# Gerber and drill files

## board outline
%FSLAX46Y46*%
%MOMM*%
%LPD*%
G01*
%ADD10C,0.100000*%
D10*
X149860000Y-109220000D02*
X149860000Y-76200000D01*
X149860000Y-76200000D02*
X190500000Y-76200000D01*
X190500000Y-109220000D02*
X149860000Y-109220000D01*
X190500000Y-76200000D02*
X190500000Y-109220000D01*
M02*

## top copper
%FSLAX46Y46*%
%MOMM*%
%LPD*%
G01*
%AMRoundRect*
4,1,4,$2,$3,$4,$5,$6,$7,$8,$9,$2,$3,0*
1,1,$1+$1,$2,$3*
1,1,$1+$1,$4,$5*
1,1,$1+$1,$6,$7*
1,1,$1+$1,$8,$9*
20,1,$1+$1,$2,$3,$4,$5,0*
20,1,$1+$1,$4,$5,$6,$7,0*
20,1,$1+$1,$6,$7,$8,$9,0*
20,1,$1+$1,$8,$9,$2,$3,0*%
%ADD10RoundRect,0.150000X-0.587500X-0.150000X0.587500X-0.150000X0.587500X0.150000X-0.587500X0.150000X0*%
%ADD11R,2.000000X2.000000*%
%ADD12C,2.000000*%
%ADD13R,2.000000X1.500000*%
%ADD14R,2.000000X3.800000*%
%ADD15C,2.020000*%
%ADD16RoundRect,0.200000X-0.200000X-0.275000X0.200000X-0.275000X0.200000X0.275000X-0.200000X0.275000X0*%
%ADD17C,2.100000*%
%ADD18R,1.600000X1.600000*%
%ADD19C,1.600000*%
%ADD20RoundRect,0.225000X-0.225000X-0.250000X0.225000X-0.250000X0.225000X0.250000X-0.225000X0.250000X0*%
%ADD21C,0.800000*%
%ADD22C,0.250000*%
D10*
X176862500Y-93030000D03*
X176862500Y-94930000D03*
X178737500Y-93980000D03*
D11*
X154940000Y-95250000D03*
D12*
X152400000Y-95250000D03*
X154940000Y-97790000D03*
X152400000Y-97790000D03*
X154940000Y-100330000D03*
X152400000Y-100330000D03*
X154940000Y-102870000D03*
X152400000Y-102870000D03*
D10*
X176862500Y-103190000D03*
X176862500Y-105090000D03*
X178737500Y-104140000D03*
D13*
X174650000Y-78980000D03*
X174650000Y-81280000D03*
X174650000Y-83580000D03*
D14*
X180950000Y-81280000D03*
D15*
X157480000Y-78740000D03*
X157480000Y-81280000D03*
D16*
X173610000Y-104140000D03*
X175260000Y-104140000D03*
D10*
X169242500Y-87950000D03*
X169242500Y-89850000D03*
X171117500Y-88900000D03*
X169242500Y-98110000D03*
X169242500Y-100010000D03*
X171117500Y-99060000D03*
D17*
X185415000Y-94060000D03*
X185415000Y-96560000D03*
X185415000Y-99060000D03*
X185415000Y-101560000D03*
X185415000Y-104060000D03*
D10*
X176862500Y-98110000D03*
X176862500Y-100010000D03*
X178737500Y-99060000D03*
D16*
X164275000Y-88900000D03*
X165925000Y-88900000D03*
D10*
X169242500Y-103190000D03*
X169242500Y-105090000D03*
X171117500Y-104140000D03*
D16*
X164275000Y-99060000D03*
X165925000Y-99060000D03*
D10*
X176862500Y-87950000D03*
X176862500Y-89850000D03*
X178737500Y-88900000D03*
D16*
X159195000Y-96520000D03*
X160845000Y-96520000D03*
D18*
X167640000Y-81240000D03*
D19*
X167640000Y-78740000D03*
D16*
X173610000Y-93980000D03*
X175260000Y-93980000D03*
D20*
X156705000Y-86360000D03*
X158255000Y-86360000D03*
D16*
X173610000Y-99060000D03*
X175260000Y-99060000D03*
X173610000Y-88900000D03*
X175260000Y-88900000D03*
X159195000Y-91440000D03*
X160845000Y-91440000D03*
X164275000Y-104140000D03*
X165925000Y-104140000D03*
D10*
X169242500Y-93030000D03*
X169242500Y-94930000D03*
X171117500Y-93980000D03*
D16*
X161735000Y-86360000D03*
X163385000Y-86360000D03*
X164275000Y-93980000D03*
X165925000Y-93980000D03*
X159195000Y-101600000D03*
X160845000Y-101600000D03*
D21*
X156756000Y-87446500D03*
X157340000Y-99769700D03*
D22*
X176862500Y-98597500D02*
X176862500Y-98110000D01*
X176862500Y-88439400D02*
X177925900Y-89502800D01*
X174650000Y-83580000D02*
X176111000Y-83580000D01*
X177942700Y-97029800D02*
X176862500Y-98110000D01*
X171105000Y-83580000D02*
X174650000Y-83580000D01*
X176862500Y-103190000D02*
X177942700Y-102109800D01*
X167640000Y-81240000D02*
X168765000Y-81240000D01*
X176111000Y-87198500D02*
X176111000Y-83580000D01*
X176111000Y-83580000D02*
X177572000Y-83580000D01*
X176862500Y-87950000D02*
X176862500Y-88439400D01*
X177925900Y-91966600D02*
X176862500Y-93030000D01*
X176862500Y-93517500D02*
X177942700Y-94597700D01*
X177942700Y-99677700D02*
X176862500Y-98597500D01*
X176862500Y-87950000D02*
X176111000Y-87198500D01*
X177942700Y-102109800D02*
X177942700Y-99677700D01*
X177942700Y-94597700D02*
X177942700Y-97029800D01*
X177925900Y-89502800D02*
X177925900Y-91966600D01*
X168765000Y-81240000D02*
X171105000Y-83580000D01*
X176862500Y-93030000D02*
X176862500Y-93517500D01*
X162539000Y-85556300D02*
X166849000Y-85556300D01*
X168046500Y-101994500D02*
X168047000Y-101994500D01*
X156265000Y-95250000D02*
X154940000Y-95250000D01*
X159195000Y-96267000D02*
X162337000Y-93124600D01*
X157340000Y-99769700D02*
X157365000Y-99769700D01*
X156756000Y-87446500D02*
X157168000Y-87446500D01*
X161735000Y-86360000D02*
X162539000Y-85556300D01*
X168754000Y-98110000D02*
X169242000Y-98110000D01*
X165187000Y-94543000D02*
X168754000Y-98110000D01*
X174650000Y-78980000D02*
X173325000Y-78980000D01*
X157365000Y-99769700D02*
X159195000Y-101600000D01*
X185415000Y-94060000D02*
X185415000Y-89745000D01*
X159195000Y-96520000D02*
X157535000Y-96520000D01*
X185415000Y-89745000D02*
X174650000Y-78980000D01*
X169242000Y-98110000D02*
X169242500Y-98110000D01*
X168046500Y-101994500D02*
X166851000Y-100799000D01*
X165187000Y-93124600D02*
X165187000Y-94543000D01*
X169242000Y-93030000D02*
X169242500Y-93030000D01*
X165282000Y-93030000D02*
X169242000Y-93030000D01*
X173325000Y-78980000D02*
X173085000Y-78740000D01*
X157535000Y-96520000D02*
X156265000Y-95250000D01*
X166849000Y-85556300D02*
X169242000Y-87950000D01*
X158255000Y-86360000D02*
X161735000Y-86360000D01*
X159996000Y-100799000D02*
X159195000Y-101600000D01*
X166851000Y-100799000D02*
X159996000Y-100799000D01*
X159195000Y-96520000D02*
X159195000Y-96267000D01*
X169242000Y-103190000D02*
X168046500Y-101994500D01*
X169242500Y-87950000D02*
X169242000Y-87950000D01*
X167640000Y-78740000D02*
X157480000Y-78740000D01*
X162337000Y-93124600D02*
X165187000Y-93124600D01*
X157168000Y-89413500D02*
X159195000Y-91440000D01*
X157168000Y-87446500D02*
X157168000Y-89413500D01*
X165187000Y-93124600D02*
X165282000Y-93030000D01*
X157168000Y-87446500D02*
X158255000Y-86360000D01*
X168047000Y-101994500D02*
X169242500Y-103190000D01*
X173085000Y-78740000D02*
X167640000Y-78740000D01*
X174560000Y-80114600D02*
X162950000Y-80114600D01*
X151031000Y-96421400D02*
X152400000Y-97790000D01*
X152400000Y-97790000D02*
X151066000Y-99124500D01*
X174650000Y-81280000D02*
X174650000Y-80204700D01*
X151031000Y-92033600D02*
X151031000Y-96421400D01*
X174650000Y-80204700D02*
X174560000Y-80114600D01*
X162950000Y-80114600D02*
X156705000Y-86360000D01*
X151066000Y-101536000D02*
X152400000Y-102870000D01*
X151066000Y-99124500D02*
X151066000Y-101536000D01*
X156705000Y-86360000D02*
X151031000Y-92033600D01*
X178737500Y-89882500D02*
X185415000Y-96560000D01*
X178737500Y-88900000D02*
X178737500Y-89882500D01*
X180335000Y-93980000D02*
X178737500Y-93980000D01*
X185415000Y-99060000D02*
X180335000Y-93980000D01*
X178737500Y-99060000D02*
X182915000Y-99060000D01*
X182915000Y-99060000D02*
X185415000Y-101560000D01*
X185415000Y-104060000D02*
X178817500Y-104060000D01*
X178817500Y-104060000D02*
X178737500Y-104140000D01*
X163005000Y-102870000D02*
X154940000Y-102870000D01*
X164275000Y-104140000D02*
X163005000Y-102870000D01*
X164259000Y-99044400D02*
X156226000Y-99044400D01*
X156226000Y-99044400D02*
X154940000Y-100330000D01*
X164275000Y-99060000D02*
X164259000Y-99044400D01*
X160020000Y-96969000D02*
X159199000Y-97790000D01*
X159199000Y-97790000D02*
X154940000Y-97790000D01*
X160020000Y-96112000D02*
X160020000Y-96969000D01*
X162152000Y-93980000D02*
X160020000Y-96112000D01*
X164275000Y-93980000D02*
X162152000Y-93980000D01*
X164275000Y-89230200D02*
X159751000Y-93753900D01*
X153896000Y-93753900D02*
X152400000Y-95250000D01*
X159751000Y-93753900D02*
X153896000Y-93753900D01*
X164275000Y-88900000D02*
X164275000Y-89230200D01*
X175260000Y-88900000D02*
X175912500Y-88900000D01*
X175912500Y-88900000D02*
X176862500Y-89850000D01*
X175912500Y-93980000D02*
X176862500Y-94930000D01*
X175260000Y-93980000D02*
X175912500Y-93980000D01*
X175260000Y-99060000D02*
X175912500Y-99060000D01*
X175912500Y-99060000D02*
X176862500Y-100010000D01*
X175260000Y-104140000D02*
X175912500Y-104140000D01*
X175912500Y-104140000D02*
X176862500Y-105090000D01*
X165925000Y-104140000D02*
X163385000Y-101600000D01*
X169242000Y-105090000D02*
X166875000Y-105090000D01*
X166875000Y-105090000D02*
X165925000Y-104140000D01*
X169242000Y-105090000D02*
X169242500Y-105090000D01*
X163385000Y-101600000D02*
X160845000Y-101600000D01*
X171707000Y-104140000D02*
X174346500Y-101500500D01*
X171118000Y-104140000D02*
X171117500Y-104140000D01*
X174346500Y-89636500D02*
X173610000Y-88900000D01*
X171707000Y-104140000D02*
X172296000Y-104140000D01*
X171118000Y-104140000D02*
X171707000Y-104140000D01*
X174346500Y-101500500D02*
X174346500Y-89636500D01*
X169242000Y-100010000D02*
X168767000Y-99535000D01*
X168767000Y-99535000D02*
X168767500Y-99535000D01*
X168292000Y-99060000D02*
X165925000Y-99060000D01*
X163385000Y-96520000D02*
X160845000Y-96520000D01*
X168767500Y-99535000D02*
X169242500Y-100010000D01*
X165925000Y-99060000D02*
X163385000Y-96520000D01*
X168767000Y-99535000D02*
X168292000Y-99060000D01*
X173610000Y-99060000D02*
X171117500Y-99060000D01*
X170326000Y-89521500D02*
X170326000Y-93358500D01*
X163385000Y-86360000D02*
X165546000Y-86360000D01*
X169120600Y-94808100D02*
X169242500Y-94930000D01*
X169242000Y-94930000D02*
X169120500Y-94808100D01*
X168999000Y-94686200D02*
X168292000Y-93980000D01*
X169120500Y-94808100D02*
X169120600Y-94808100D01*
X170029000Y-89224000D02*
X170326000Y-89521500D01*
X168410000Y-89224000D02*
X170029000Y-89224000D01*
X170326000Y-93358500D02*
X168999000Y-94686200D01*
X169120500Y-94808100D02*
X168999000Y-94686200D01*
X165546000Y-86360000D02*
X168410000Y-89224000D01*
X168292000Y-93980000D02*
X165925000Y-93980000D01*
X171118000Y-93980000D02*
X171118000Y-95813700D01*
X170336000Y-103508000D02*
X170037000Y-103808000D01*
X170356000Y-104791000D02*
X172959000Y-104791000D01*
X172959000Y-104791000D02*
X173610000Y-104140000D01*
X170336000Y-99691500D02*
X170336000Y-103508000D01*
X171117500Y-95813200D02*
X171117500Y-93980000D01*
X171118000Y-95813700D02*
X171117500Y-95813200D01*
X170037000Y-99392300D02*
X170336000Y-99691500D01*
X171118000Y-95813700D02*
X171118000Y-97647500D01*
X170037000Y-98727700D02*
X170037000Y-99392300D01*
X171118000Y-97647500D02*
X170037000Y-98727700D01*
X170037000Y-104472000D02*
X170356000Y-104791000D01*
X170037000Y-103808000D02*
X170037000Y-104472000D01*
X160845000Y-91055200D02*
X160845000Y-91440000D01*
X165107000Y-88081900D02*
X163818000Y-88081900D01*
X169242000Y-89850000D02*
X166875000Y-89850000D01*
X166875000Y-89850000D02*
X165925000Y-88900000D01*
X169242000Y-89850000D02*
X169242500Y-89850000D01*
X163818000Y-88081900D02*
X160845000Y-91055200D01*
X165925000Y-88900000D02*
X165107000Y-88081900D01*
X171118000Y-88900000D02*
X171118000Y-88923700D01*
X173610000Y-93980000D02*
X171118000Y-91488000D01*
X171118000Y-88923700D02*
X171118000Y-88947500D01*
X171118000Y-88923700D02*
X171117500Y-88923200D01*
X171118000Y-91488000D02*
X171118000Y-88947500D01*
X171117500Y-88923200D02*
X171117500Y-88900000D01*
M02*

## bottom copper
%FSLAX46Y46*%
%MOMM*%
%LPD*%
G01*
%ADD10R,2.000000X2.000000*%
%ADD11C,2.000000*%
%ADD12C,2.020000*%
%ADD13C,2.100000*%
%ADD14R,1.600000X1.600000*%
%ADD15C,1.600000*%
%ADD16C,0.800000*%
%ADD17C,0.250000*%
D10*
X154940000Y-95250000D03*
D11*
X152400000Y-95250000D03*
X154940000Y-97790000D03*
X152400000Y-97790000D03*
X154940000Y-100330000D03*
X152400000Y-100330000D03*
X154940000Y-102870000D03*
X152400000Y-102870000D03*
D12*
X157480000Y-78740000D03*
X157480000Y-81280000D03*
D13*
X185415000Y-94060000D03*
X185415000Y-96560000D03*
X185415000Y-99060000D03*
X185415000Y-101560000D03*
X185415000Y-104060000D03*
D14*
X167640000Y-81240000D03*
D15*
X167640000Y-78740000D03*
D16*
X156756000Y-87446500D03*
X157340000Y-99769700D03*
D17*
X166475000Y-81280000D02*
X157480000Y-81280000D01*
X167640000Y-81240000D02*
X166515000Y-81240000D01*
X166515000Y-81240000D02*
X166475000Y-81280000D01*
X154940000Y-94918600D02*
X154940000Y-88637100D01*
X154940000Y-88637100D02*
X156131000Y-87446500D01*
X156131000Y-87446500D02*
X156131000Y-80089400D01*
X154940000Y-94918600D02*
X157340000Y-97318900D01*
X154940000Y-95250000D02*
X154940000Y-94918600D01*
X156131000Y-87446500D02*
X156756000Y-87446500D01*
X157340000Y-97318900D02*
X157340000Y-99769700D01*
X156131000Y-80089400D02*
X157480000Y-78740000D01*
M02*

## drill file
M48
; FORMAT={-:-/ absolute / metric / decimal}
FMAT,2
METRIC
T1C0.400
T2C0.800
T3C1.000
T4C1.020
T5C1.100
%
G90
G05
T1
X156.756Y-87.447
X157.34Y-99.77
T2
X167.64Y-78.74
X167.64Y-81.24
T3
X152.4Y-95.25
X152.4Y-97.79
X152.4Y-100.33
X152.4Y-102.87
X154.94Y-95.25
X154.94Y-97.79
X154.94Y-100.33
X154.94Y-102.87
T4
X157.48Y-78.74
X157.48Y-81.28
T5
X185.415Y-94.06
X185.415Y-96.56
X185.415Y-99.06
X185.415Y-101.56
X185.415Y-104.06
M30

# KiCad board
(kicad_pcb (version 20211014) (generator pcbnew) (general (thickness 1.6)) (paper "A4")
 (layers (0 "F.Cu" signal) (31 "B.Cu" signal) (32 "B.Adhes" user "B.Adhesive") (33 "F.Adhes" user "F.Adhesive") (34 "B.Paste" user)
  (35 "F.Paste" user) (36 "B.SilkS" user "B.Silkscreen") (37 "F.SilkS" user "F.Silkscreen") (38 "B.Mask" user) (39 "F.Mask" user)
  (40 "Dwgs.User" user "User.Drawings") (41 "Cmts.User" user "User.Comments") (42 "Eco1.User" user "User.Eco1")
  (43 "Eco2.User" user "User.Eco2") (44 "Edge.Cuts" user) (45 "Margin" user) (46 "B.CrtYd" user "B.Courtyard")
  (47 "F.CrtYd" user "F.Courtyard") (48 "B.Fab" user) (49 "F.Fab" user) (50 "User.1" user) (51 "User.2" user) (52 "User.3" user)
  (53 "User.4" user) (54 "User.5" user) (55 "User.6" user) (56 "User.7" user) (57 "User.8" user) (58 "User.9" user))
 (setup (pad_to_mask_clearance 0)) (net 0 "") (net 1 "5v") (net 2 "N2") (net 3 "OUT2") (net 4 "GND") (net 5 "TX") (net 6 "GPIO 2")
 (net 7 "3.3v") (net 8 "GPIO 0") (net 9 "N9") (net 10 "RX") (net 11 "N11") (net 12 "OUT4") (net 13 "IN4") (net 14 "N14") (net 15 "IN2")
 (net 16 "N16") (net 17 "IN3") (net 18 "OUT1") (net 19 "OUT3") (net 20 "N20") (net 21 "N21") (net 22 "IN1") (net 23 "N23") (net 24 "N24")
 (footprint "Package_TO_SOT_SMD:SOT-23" (layer "F.Cu") (at 177.8 93.98)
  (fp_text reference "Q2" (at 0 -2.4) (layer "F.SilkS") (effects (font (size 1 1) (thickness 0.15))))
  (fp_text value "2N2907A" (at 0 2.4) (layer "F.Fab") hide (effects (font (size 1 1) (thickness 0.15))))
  (pad "1" smd roundrect (at -0.9375 -0.95) (size 1.475 0.6) (layers "F.Cu" "F.Paste" "F.Mask") (roundrect_rratio 0.25) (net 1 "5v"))
  (pad "2" smd roundrect (at -0.9375 0.95) (size 1.475 0.6) (layers "F.Cu" "F.Paste" "F.Mask") (roundrect_rratio 0.25) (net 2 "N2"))
  (pad "3" smd roundrect (at 0.9375 0) (size 1.475 0.6) (layers "F.Cu" "F.Paste" "F.Mask") (roundrect_rratio 0.25) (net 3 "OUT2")))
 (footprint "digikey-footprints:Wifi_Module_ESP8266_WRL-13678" (layer "F.Cu") (at 154.94 95.25 -90)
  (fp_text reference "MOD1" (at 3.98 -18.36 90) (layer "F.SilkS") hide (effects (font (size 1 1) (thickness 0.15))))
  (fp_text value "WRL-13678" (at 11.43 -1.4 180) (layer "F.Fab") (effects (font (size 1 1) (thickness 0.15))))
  (pad "1" thru_hole rect (at 0 0 90) (size 2 2) (drill 1) (layers *.Cu *.Mask) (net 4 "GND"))
  (pad "2" thru_hole circle (at 0 2.54 90) (size 2 2) (drill 1) (layers *.Cu *.Mask) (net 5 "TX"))
  (pad "3" thru_hole circle (at 2.54 0 90) (size 2 2) (drill 1) (layers *.Cu *.Mask) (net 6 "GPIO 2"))
  (pad "4" thru_hole circle (at 2.54 2.54 90) (size 2 2) (drill 1) (layers *.Cu *.Mask) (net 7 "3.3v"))
  (pad "5" thru_hole circle (at 5.08 0 90) (size 2 2) (drill 1) (layers *.Cu *.Mask) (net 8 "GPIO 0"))
  (pad "6" thru_hole circle (at 5.08 2.54 90) (size 2 2) (drill 1) (layers *.Cu *.Mask) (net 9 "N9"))
  (pad "7" thru_hole circle (at 7.62 0 90) (size 2 2) (drill 1) (layers *.Cu *.Mask) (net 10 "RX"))
  (pad "8" thru_hole circle (at 7.62 2.54 90) (size 2 2) (drill 1) (layers *.Cu *.Mask) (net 7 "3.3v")))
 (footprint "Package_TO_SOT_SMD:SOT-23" (layer "F.Cu") (at 177.8 104.14)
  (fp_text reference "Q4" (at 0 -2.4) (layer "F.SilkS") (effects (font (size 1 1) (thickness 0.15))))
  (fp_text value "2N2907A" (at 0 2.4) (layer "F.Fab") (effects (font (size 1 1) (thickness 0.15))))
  (pad "1" smd roundrect (at -0.9375 -0.95) (size 1.475 0.6) (layers "F.Cu" "F.Paste" "F.Mask") (roundrect_rratio 0.25) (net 1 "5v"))
  (pad "2" smd roundrect (at -0.9375 0.95) (size 1.475 0.6) (layers "F.Cu" "F.Paste" "F.Mask") (roundrect_rratio 0.25) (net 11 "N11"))
  (pad "3" smd roundrect (at 0.9375 0) (size 1.475 0.6) (layers "F.Cu" "F.Paste" "F.Mask") (roundrect_rratio 0.25) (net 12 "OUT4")))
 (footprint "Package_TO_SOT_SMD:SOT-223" (layer "F.Cu") (at 177.8 81.28)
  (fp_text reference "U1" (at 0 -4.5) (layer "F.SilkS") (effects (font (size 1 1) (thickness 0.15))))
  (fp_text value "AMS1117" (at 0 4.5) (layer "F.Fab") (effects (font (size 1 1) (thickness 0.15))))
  (pad "1" smd rect (at -3.15 -2.3) (size 2 1.5) (layers "F.Cu" "F.Paste" "F.Mask") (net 4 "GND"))
  (pad "2" smd rect (at -3.15 0) (size 2 1.5) (layers "F.Cu" "F.Paste" "F.Mask") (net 7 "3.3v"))
  (pad "3" smd rect (at -3.15 2.3) (size 2 1.5) (layers "F.Cu" "F.Paste" "F.Mask") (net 1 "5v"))
  (pad "4" smd rect (at 3.15 0) (size 2 3.8) (layers "F.Cu" "F.Paste" "F.Mask")))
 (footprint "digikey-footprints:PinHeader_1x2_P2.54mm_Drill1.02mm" (layer "F.Cu") (at 157.48 78.74 -90)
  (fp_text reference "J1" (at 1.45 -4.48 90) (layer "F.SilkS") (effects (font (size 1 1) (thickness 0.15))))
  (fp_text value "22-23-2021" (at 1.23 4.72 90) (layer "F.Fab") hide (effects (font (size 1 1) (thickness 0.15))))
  (pad "1" thru_hole circle locked (at 0 0 270) (size 2.02 2.02) (drill 1.02) (layers *.Cu *.Mask) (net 4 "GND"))
  (pad "2" thru_hole circle locked (at 2.54 0 270) (size 2.02 2.02) (drill 1.02) (layers *.Cu *.Mask) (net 1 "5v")))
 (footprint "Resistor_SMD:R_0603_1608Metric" (layer "F.Cu") (at 174.435 104.14)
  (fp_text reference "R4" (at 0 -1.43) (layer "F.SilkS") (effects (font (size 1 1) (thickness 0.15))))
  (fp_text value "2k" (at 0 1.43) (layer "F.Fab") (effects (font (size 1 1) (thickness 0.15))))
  (pad "1" smd roundrect (at -0.825 0) (size 0.8 0.95) (layers "F.Cu" "F.Paste" "F.Mask") (roundrect_rratio 0.25) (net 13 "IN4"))
  (pad "2" smd roundrect (at 0.825 0) (size 0.8 0.95) (layers "F.Cu" "F.Paste" "F.Mask") (roundrect_rratio 0.25) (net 11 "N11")))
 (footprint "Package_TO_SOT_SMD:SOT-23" (layer "F.Cu") (at 170.18 88.9)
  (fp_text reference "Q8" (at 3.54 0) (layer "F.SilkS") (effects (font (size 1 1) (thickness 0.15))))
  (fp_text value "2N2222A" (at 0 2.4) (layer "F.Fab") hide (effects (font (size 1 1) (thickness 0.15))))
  (pad "1" smd roundrect (at -0.9375 -0.95) (size 1.475 0.6) (layers "F.Cu" "F.Paste" "F.Mask") (roundrect_rratio 0.25) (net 4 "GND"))
  (pad "2" smd roundrect (at -0.9375 0.95) (size 1.475 0.6) (layers "F.Cu" "F.Paste" "F.Mask") (roundrect_rratio 0.25) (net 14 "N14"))
  (pad "3" smd roundrect (at 0.9375 0) (size 1.475 0.6) (layers "F.Cu" "F.Paste" "F.Mask") (roundrect_rratio 0.25) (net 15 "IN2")))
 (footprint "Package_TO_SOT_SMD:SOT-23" (layer "F.Cu") (at 170.18 99.06)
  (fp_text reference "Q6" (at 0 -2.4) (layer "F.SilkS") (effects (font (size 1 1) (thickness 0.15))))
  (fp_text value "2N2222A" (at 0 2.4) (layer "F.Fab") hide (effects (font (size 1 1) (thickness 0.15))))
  (pad "1" smd roundrect (at -0.9375 -0.95) (size 1.475 0.6) (layers "F.Cu" "F.Paste" "F.Mask") (roundrect_rratio 0.25) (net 4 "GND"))
  (pad "2" smd roundrect (at -0.9375 0.95) (size 1.475 0.6) (layers "F.Cu" "F.Paste" "F.Mask") (roundrect_rratio 0.25) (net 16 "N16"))
  (pad "3" smd roundrect (at 0.9375 0) (size 1.475 0.6) (layers "F.Cu" "F.Paste" "F.Mask") (roundrect_rratio 0.25) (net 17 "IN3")))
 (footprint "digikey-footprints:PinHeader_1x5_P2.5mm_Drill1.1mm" (layer "F.Cu") (at 185.415 94.06 -90)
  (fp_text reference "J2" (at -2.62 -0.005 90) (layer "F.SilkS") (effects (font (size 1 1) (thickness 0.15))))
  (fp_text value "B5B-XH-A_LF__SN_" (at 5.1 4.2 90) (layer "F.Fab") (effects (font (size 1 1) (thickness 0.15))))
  (pad "1" thru_hole circle locked (at 0 0 270) (size 2.1 2.1) (drill 1.1) (layers *.Cu *.Mask) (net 4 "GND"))
  (pad "2" thru_hole circle locked (at 2.5 0 270) (size 2.1 2.1) (drill 1.1) (layers *.Cu *.Mask) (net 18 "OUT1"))
  (pad "3" thru_hole circle locked (at 5 0 270) (size 2.1 2.1) (drill 1.1) (layers *.Cu *.Mask) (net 3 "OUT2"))
  (pad "4" thru_hole circle locked (at 7.5 0 270) (size 2.1 2.1) (drill 1.1) (layers *.Cu *.Mask) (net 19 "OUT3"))
  (pad "5" thru_hole circle locked (at 10 0 270) (size 2.1 2.1) (drill 1.1) (layers *.Cu *.Mask) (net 12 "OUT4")))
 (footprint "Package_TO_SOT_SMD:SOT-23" (layer "F.Cu") (at 177.8 99.06)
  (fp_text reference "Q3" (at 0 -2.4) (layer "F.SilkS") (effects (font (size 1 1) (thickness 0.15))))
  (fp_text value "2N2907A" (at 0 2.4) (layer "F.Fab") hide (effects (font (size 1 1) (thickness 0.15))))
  (pad "1" smd roundrect (at -0.9375 -0.95) (size 1.475 0.6) (layers "F.Cu" "F.Paste" "F.Mask") (roundrect_rratio 0.25) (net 1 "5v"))
  (pad "2" smd roundrect (at -0.9375 0.95) (size 1.475 0.6) (layers "F.Cu" "F.Paste" "F.Mask") (roundrect_rratio 0.25) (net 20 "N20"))
  (pad "3" smd roundrect (at 0.9375 0) (size 1.475 0.6) (layers "F.Cu" "F.Paste" "F.Mask") (roundrect_rratio 0.25) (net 19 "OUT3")))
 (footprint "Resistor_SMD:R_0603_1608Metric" (layer "F.Cu") (at 165.1 88.9)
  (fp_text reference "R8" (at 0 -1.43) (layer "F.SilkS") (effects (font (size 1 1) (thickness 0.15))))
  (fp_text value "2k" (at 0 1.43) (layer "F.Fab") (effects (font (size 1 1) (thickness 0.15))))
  (pad "1" smd roundrect (at -0.825 0) (size 0.8 0.95) (layers "F.Cu" "F.Paste" "F.Mask") (roundrect_rratio 0.25) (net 5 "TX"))
  (pad "2" smd roundrect (at 0.825 0) (size 0.8 0.95) (layers "F.Cu" "F.Paste" "F.Mask") (roundrect_rratio 0.25) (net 14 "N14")))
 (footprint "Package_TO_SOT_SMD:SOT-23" (layer "F.Cu") (at 170.18 104.14)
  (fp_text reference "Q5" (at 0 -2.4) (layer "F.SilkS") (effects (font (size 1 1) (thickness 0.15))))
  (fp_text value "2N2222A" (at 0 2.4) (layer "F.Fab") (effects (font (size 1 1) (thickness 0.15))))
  (pad "1" smd roundrect (at -0.9375 -0.95) (size 1.475 0.6) (layers "F.Cu" "F.Paste" "F.Mask") (roundrect_rratio 0.25) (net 4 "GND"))
  (pad "2" smd roundrect (at -0.9375 0.95) (size 1.475 0.6) (layers "F.Cu" "F.Paste" "F.Mask") (roundrect_rratio 0.25) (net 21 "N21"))
  (pad "3" smd roundrect (at 0.9375 0) (size 1.475 0.6) (layers "F.Cu" "F.Paste" "F.Mask") (roundrect_rratio 0.25) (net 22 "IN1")))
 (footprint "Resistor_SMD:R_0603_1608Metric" (layer "F.Cu") (at 165.1 99.06)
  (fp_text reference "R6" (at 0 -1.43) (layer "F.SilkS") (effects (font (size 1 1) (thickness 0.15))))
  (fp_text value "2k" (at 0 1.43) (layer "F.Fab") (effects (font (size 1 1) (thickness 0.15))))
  (pad "1" smd roundrect (at -0.825 0) (size 0.8 0.95) (layers "F.Cu" "F.Paste" "F.Mask") (roundrect_rratio 0.25) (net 8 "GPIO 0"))
  (pad "2" smd roundrect (at 0.825 0) (size 0.8 0.95) (layers "F.Cu" "F.Paste" "F.Mask") (roundrect_rratio 0.25) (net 16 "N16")))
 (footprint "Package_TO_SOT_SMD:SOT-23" (layer "F.Cu") (at 177.8 88.9)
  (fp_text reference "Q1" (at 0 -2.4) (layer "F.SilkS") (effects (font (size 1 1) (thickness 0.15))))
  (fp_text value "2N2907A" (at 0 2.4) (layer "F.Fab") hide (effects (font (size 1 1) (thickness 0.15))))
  (pad "1" smd roundrect (at -0.9375 -0.95) (size 1.475 0.6) (layers "F.Cu" "F.Paste" "F.Mask") (roundrect_rratio 0.25) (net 1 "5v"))
  (pad "2" smd roundrect (at -0.9375 0.95) (size 1.475 0.6) (layers "F.Cu" "F.Paste" "F.Mask") (roundrect_rratio 0.25) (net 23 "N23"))
  (pad "3" smd roundrect (at 0.9375 0) (size 1.475 0.6) (layers "F.Cu" "F.Paste" "F.Mask") (roundrect_rratio 0.25) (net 18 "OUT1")))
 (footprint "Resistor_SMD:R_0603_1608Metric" (layer "F.Cu") (at 160.02 96.52)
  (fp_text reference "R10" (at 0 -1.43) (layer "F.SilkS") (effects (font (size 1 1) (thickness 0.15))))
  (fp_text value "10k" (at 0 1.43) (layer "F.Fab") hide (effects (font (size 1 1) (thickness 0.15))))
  (pad "1" smd roundrect (at -0.825 0) (size 0.8 0.95) (layers "F.Cu" "F.Paste" "F.Mask") (roundrect_rratio 0.25) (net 4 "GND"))
  (pad "2" smd roundrect (at 0.825 0) (size 0.8 0.95) (layers "F.Cu" "F.Paste" "F.Mask") (roundrect_rratio 0.25) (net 16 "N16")))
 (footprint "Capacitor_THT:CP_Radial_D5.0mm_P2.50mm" (layer "F.Cu") (at 167.64 81.24 90)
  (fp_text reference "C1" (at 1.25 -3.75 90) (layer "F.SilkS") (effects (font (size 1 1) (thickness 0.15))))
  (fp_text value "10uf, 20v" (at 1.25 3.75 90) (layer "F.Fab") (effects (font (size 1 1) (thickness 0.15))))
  (pad "1" thru_hole rect (at 0 0 90) (size 1.6 1.6) (drill 0.8) (layers *.Cu *.Mask) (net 1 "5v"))
  (pad "2" thru_hole circle (at 2.5 0 90) (size 1.6 1.6) (drill 0.8) (layers *.Cu *.Mask) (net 4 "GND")))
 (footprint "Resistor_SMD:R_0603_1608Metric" (layer "F.Cu") (at 174.435 93.98)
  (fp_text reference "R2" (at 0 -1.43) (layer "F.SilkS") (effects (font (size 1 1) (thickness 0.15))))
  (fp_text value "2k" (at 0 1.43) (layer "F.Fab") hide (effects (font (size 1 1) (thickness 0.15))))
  (pad "1" smd roundrect (at -0.825 0) (size 0.8 0.95) (layers "F.Cu" "F.Paste" "F.Mask") (roundrect_rratio 0.25) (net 15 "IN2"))
  (pad "2" smd roundrect (at 0.825 0) (size 0.8 0.95) (layers "F.Cu" "F.Paste" "F.Mask") (roundrect_rratio 0.25) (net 2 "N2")))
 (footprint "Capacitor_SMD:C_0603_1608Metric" (layer "F.Cu") (at 157.48 86.36)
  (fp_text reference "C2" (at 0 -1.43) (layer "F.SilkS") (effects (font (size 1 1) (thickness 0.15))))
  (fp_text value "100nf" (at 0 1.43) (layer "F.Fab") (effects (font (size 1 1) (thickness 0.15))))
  (pad "1" smd roundrect (at -0.775 0) (size 0.9 0.95) (layers "F.Cu" "F.Paste" "F.Mask") (roundrect_rratio 0.25) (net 7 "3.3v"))
  (pad "2" smd roundrect (at 0.775 0) (size 0.9 0.95) (layers "F.Cu" "F.Paste" "F.Mask") (roundrect_rratio 0.25) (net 4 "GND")))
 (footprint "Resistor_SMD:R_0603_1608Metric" (layer "F.Cu") (at 174.435 99.06)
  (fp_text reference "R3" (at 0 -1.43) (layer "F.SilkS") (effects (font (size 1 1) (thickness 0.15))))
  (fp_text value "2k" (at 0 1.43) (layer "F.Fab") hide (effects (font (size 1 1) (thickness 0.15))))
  (pad "1" smd roundrect (at -0.825 0) (size 0.8 0.95) (layers "F.Cu" "F.Paste" "F.Mask") (roundrect_rratio 0.25) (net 17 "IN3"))
  (pad "2" smd roundrect (at 0.825 0) (size 0.8 0.95) (layers "F.Cu" "F.Paste" "F.Mask") (roundrect_rratio 0.25) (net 20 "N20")))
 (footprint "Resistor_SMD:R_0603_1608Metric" (layer "F.Cu") (at 174.435 88.9)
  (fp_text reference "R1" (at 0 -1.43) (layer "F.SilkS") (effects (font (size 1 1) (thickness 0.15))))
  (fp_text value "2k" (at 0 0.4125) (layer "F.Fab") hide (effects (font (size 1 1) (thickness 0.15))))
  (pad "1" smd roundrect (at -0.825 0) (size 0.8 0.95) (layers "F.Cu" "F.Paste" "F.Mask") (roundrect_rratio 0.25) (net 22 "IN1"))
  (pad "2" smd roundrect (at 0.825 0) (size 0.8 0.95) (layers "F.Cu" "F.Paste" "F.Mask") (roundrect_rratio 0.25) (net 23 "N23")))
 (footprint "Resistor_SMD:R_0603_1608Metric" (layer "F.Cu") (at 160.02 91.44)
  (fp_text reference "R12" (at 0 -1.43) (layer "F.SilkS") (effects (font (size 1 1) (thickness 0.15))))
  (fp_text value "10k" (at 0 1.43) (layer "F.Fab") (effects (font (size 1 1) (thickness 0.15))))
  (pad "1" smd roundrect (at -0.825 0) (size 0.8 0.95) (layers "F.Cu" "F.Paste" "F.Mask") (roundrect_rratio 0.25) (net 4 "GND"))
  (pad "2" smd roundrect (at 0.825 0) (size 0.8 0.95) (layers "F.Cu" "F.Paste" "F.Mask") (roundrect_rratio 0.25) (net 14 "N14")))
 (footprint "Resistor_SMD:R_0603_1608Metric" (layer "F.Cu") (at 165.1 104.14)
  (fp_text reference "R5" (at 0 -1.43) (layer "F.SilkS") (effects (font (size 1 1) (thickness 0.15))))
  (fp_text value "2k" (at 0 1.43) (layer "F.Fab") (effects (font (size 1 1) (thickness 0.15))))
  (pad "1" smd roundrect (at -0.825 0) (size 0.8 0.95) (layers "F.Cu" "F.Paste" "F.Mask") (roundrect_rratio 0.25) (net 10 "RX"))
  (pad "2" smd roundrect (at 0.825 0) (size 0.8 0.95) (layers "F.Cu" "F.Paste" "F.Mask") (roundrect_rratio 0.25) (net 21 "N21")))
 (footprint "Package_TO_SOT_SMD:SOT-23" (layer "F.Cu") (at 170.18 93.98)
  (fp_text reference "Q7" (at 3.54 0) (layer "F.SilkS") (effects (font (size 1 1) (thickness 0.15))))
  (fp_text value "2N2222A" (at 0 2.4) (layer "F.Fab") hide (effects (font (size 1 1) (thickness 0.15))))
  (pad "1" smd roundrect (at -0.9375 -0.95) (size 1.475 0.6) (layers "F.Cu" "F.Paste" "F.Mask") (roundrect_rratio 0.25) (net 4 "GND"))
  (pad "2" smd roundrect (at -0.9375 0.95) (size 1.475 0.6) (layers "F.Cu" "F.Paste" "F.Mask") (roundrect_rratio 0.25) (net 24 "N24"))
  (pad "3" smd roundrect (at 0.9375 0) (size 1.475 0.6) (layers "F.Cu" "F.Paste" "F.Mask") (roundrect_rratio 0.25) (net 13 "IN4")))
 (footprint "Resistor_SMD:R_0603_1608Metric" (layer "F.Cu") (at 162.56 86.36)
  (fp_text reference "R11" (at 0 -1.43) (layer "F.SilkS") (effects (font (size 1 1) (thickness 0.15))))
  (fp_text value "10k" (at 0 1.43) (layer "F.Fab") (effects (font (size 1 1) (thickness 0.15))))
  (pad "1" smd roundrect (at -0.825 0) (size 0.8 0.95) (layers "F.Cu" "F.Paste" "F.Mask") (roundrect_rratio 0.25) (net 4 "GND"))
  (pad "2" smd roundrect (at 0.825 0) (size 0.8 0.95) (layers "F.Cu" "F.Paste" "F.Mask") (roundrect_rratio 0.25) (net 24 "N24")))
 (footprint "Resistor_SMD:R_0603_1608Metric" (layer "F.Cu") (at 165.1 93.98)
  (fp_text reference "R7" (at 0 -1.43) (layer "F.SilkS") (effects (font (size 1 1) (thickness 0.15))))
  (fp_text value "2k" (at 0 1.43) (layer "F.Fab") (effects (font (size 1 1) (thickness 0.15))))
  (pad "1" smd roundrect (at -0.825 0) (size 0.8 0.95) (layers "F.Cu" "F.Paste" "F.Mask") (roundrect_rratio 0.25) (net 6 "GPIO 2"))
  (pad "2" smd roundrect (at 0.825 0) (size 0.8 0.95) (layers "F.Cu" "F.Paste" "F.Mask") (roundrect_rratio 0.25) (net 24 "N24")))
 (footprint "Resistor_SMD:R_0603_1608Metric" (layer "F.Cu") (at 160.02 101.6)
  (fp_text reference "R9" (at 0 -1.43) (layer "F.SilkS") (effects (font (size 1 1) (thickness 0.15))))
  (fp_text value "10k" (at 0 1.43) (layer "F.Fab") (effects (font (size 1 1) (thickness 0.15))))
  (pad "1" smd roundrect (at -0.825 0) (size 0.8 0.95) (layers "F.Cu" "F.Paste" "F.Mask") (roundrect_rratio 0.25) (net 4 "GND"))
  (pad "2" smd roundrect (at 0.825 0) (size 0.8 0.95) (layers "F.Cu" "F.Paste" "F.Mask") (roundrect_rratio 0.25) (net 21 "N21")))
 (gr_line (start 149.86 109.22) (end 149.86 76.2) (layer "Edge.Cuts") (width 0.1))
 (gr_line (start 149.86 76.2) (end 190.5 76.2) (layer "Edge.Cuts") (width 0.1))
 (gr_line (start 190.5 109.22) (end 149.86 109.22) (layer "Edge.Cuts") (width 0.1))
 (gr_line (start 190.5 76.2) (end 190.5 109.22) (layer "Edge.Cuts") (width 0.1))
 (segment (start 176.8625 98.5975) (end 176.8625 98.11) (width 0.25) (layer "F.Cu") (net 1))
 (segment (start 176.8625 88.4394) (end 177.9259 89.5028) (width 0.25) (layer "F.Cu") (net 1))
 (segment (start 174.65 83.58) (end 176.111 83.58) (width 0.25) (layer "F.Cu") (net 1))
 (segment (start 177.9427 97.0298) (end 176.8625 98.11) (width 0.25) (layer "F.Cu") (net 1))
 (segment (start 171.105 83.58) (end 174.65 83.58) (width 0.25) (layer "F.Cu") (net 1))
 (segment (start 176.8625 103.19) (end 177.9427 102.1098) (width 0.25) (layer "F.Cu") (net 1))
 (segment (start 167.64 81.24) (end 168.765 81.24) (width 0.25) (layer "F.Cu") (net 1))
 (segment (start 176.111 87.1985) (end 176.111 83.58) (width 0.25) (layer "F.Cu") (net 1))
 (segment (start 176.111 83.58) (end 177.572 83.58) (width 0.25) (layer "F.Cu") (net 1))
 (segment (start 176.8625 87.95) (end 176.8625 88.4394) (width 0.25) (layer "F.Cu") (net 1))
 (segment (start 177.9259 91.9666) (end 176.8625 93.03) (width 0.25) (layer "F.Cu") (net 1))
 (segment (start 176.8625 93.5175) (end 177.9427 94.5977) (width 0.25) (layer "F.Cu") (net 1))
 (segment (start 177.9427 99.6777) (end 176.8625 98.5975) (width 0.25) (layer "F.Cu") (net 1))
 (segment (start 176.8625 87.95) (end 176.111 87.1985) (width 0.25) (layer "F.Cu") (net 1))
 (segment (start 177.9427 102.1098) (end 177.9427 99.6777) (width 0.25) (layer "F.Cu") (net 1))
 (segment (start 177.9427 94.5977) (end 177.9427 97.0298) (width 0.25) (layer "F.Cu") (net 1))
 (segment (start 177.9259 89.5028) (end 177.9259 91.9666) (width 0.25) (layer "F.Cu") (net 1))
 (segment (start 168.765 81.24) (end 171.105 83.58) (width 0.25) (layer "F.Cu") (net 1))
 (segment (start 176.8625 93.03) (end 176.8625 93.5175) (width 0.25) (layer "F.Cu") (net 1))
 (segment (start 166.475 81.28) (end 157.48 81.28) (width 0.25) (layer "B.Cu") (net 1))
 (segment (start 167.64 81.24) (end 166.515 81.24) (width 0.25) (layer "B.Cu") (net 1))
 (segment (start 166.515 81.24) (end 166.475 81.28) (width 0.25) (layer "B.Cu") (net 1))
 (segment (start 162.539 85.5563) (end 166.849 85.5563) (width 0.25) (layer "F.Cu") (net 4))
 (segment (start 168.0465 101.9945) (end 168.047 101.9945) (width 0.25) (layer "F.Cu") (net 4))
 (segment (start 156.265 95.25) (end 154.94 95.25) (width 0.25) (layer "F.Cu") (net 4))
 (segment (start 159.195 96.267) (end 162.337 93.1246) (width 0.25) (layer "F.Cu") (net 4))
 (segment (start 157.34 99.7697) (end 157.365 99.7697) (width 0.25) (layer "F.Cu") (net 4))
 (segment (start 156.756 87.4465) (end 157.168 87.4465) (width 0.25) (layer "F.Cu") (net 4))
 (segment (start 161.735 86.36) (end 162.539 85.5563) (width 0.25) (layer "F.Cu") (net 4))
 (segment (start 168.754 98.11) (end 169.242 98.11) (width 0.25) (layer "F.Cu") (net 4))
 (segment (start 165.187 94.543) (end 168.754 98.11) (width 0.25) (layer "F.Cu") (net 4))
 (segment (start 174.65 78.98) (end 173.325 78.98) (width 0.25) (layer "F.Cu") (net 4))
 (segment (start 157.365 99.7697) (end 159.195 101.6) (width 0.25) (layer "F.Cu") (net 4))
 (segment (start 185.415 94.06) (end 185.415 89.745) (width 0.25) (layer "F.Cu") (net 4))
 (segment (start 159.195 96.52) (end 157.535 96.52) (width 0.25) (layer "F.Cu") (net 4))
 (segment (start 185.415 89.745) (end 174.65 78.98) (width 0.25) (layer "F.Cu") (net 4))
 (segment (start 169.242 98.11) (end 169.2425 98.11) (width 0.25) (layer "F.Cu") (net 4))
 (segment (start 168.0465 101.9945) (end 166.851 100.799) (width 0.25) (layer "F.Cu") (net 4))
 (segment (start 165.187 93.1246) (end 165.187 94.543) (width 0.25) (layer "F.Cu") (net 4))
 (segment (start 169.242 93.03) (end 169.2425 93.03) (width 0.25) (layer "F.Cu") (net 4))
 (segment (start 165.282 93.03) (end 169.242 93.03) (width 0.25) (layer "F.Cu") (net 4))
 (segment (start 173.325 78.98) (end 173.085 78.74) (width 0.25) (layer "F.Cu") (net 4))
 (segment (start 157.535 96.52) (end 156.265 95.25) (width 0.25) (layer "F.Cu") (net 4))
 (segment (start 166.849 85.5563) (end 169.242 87.95) (width 0.25) (layer "F.Cu") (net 4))
 (segment (start 158.255 86.36) (end 161.735 86.36) (width 0.25) (layer "F.Cu") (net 4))
 (segment (start 159.996 100.799) (end 159.195 101.6) (width 0.25) (layer "F.Cu") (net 4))
 (segment (start 166.851 100.799) (end 159.996 100.799) (width 0.25) (layer "F.Cu") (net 4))
 (segment (start 159.195 96.52) (end 159.195 96.267) (width 0.25) (layer "F.Cu") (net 4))
 (segment (start 169.242 103.19) (end 168.0465 101.9945) (width 0.25) (layer "F.Cu") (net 4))
 (segment (start 169.2425 87.95) (end 169.242 87.95) (width 0.25) (layer "F.Cu") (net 4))
 (segment (start 167.64 78.74) (end 157.48 78.74) (width 0.25) (layer "F.Cu") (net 4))
 (segment (start 162.337 93.1246) (end 165.187 93.1246) (width 0.25) (layer "F.Cu") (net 4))
 (segment (start 157.168 89.4135) (end 159.195 91.44) (width 0.25) (layer "F.Cu") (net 4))
 (segment (start 157.168 87.4465) (end 157.168 89.4135) (width 0.25) (layer "F.Cu") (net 4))
 (segment (start 165.187 93.1246) (end 165.282 93.03) (width 0.25) (layer "F.Cu") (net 4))
 (segment (start 157.168 87.4465) (end 158.255 86.36) (width 0.25) (layer "F.Cu") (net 4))
 (segment (start 168.047 101.9945) (end 169.2425 103.19) (width 0.25) (layer "F.Cu") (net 4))
 (segment (start 173.085 78.74) (end 167.64 78.74) (width 0.25) (layer "F.Cu") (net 4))
 (via (at 156.756 87.4465) (size 0.8) (drill 0.4) (layers "F.Cu" "B.Cu") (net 4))
 (via (at 157.34 99.7697) (size 0.8) (drill 0.4) (layers "F.Cu" "B.Cu") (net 4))
 (segment (start 154.94 94.9186) (end 154.94 88.6371) (width 0.25) (layer "B.Cu") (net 4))
 (segment (start 154.94 88.6371) (end 156.131 87.4465) (width 0.25) (layer "B.Cu") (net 4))
 (segment (start 156.131 87.4465) (end 156.131 80.0894) (width 0.25) (layer "B.Cu") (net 4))
 (segment (start 154.94 94.9186) (end 157.34 97.3189) (width 0.25) (layer "B.Cu") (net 4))
 (segment (start 154.94 95.25) (end 154.94 94.9186) (width 0.25) (layer "B.Cu") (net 4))
 (segment (start 156.131 87.4465) (end 156.756 87.4465) (width 0.25) (layer "B.Cu") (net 4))
 (segment (start 157.34 97.3189) (end 157.34 99.7697) (width 0.25) (layer "B.Cu") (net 4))
 (segment (start 156.131 80.0894) (end 157.48 78.74) (width 0.25) (layer "B.Cu") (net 4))
 (segment (start 174.56 80.1146) (end 162.95 80.1146) (width 0.25) (layer "F.Cu") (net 7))
 (segment (start 151.031 96.4214) (end 152.4 97.79) (width 0.25) (layer "F.Cu") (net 7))
 (segment (start 152.4 97.79) (end 151.066 99.1245) (width 0.25) (layer "F.Cu") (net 7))
 (segment (start 174.65 81.28) (end 174.65 80.2047) (width 0.25) (layer "F.Cu") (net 7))
 (segment (start 151.031 92.0336) (end 151.031 96.4214) (width 0.25) (layer "F.Cu") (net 7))
 (segment (start 174.65 80.2047) (end 174.56 80.1146) (width 0.25) (layer "F.Cu") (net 7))
 (segment (start 162.95 80.1146) (end 156.705 86.36) (width 0.25) (layer "F.Cu") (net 7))
 (segment (start 151.066 101.536) (end 152.4 102.87) (width 0.25) (layer "F.Cu") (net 7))
 (segment (start 151.066 99.1245) (end 151.066 101.536) (width 0.25) (layer "F.Cu") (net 7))
 (segment (start 156.705 86.36) (end 151.031 92.0336) (width 0.25) (layer "F.Cu") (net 7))
 (segment (start 178.7375 89.8825) (end 185.415 96.56) (width 0.25) (layer "F.Cu") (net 18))
 (segment (start 178.7375 88.9) (end 178.7375 89.8825) (width 0.25) (layer "F.Cu") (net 18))
 (segment (start 180.335 93.98) (end 178.7375 93.98) (width 0.25) (layer "F.Cu") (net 3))
 (segment (start 185.415 99.06) (end 180.335 93.98) (width 0.25) (layer "F.Cu") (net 3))
 (segment (start 178.7375 99.06) (end 182.915 99.06) (width 0.25) (layer "F.Cu") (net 19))
 (segment (start 182.915 99.06) (end 185.415 101.56) (width 0.25) (layer "F.Cu") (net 19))
 (segment (start 185.415 104.06) (end 178.8175 104.06) (width 0.25) (layer "F.Cu") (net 12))
 (segment (start 178.8175 104.06) (end 178.7375 104.14) (width 0.25) (layer "F.Cu") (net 12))
 (segment (start 163.005 102.87) (end 154.94 102.87) (width 0.25) (layer "F.Cu") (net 10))
 (segment (start 164.275 104.14) (end 163.005 102.87) (width 0.25) (layer "F.Cu") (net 10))
 (segment (start 164.259 99.0444) (end 156.226 99.0444) (width 0.25) (layer "F.Cu") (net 8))
 (segment (start 156.226 99.0444) (end 154.94 100.33) (width 0.25) (layer "F.Cu") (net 8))
 (segment (start 164.275 99.06) (end 164.259 99.0444) (width 0.25) (layer "F.Cu") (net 8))
 (segment (start 160.02 96.969) (end 159.199 97.79) (width 0.25) (layer "F.Cu") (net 6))
 (segment (start 159.199 97.79) (end 154.94 97.79) (width 0.25) (layer "F.Cu") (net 6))
 (segment (start 160.02 96.112) (end 160.02 96.969) (width 0.25) (layer "F.Cu") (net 6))
 (segment (start 162.152 93.98) (end 160.02 96.112) (width 0.25) (layer "F.Cu") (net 6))
 (segment (start 164.275 93.98) (end 162.152 93.98) (width 0.25) (layer "F.Cu") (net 6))
 (segment (start 164.275 89.2302) (end 159.751 93.7539) (width 0.25) (layer "F.Cu") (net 5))
 (segment (start 153.896 93.7539) (end 152.4 95.25) (width 0.25) (layer "F.Cu") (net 5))
 (segment (start 159.751 93.7539) (end 153.896 93.7539) (width 0.25) (layer "F.Cu") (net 5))
 (segment (start 164.275 88.9) (end 164.275 89.2302) (width 0.25) (layer "F.Cu") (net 5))
 (segment (start 175.26 88.9) (end 175.9125 88.9) (width 0.25) (layer "F.Cu") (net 23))
 (segment (start 175.9125 88.9) (end 176.8625 89.85) (width 0.25) (layer "F.Cu") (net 23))
 (segment (start 175.9125 93.98) (end 176.8625 94.93) (width 0.25) (layer "F.Cu") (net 2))
 (segment (start 175.26 93.98) (end 175.9125 93.98) (width 0.25) (layer "F.Cu") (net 2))
 (segment (start 175.26 99.06) (end 175.9125 99.06) (width 0.25) (layer "F.Cu") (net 20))
 (segment (start 175.9125 99.06) (end 176.8625 100.01) (width 0.25) (layer "F.Cu") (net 20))
 (segment (start 175.26 104.14) (end 175.9125 104.14) (width 0.25) (layer "F.Cu") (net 11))
 (segment (start 175.9125 104.14) (end 176.8625 105.09) (width 0.25) (layer "F.Cu") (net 11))
 (segment (start 165.925 104.14) (end 163.385 101.6) (width 0.25) (layer "F.Cu") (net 21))
 (segment (start 169.242 105.09) (end 166.875 105.09) (width 0.25) (layer "F.Cu") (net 21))
 (segment (start 166.875 105.09) (end 165.925 104.14) (width 0.25) (layer "F.Cu") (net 21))
 (segment (start 169.242 105.09) (end 169.2425 105.09) (width 0.25) (layer "F.Cu") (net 21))
 (segment (start 163.385 101.6) (end 160.845 101.6) (width 0.25) (layer "F.Cu") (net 21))
 (segment (start 171.707 104.14) (end 174.3465 101.5005) (width 0.25) (layer "F.Cu") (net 22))
 (segment (start 171.118 104.14) (end 171.1175 104.14) (width 0.25) (layer "F.Cu") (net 22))
 (segment (start 174.3465 89.6365) (end 173.61 88.9) (width 0.25) (layer "F.Cu") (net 22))
 (segment (start 171.707 104.14) (end 172.296 104.14) (width 0.25) (layer "F.Cu") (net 22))
 (segment (start 171.118 104.14) (end 171.707 104.14) (width 0.25) (layer "F.Cu") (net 22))
 (segment (start 174.3465 101.5005) (end 174.3465 89.6365) (width 0.25) (layer "F.Cu") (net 22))
 (segment (start 169.242 100.01) (end 168.767 99.535) (width 0.25) (layer "F.Cu") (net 16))
 (segment (start 168.767 99.535) (end 168.7675 99.535) (width 0.25) (layer "F.Cu") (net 16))
 (segment (start 168.292 99.06) (end 165.925 99.06) (width 0.25) (layer "F.Cu") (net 16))
 (segment (start 163.385 96.52) (end 160.845 96.52) (width 0.25) (layer "F.Cu") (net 16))
 (segment (start 168.7675 99.535) (end 169.2425 100.01) (width 0.25) (layer "F.Cu") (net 16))
 (segment (start 165.925 99.06) (end 163.385 96.52) (width 0.25) (layer "F.Cu") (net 16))
 (segment (start 168.767 99.535) (end 168.292 99.06) (width 0.25) (layer "F.Cu") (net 16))
 (segment (start 173.61 99.06) (end 171.1175 99.06) (width 0.25) (layer "F.Cu") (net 17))
 (segment (start 170.326 89.5215) (end 170.326 93.3585) (width 0.25) (layer "F.Cu") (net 24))
 (segment (start 163.385 86.36) (end 165.546 86.36) (width 0.25) (layer "F.Cu") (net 24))
 (segment (start 169.1206 94.8081) (end 169.2425 94.93) (width 0.25) (layer "F.Cu") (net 24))
 (segment (start 169.242 94.93) (end 169.1205 94.8081) (width 0.25) (layer "F.Cu") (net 24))
 (segment (start 168.999 94.6862) (end 168.292 93.98) (width 0.25) (layer "F.Cu") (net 24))
 (segment (start 169.1205 94.8081) (end 169.1206 94.8081) (width 0.25) (layer "F.Cu") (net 24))
 (segment (start 170.029 89.224) (end 170.326 89.5215) (width 0.25) (layer "F.Cu") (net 24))
 (segment (start 168.41 89.224) (end 170.029 89.224) (width 0.25) (layer "F.Cu") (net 24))
 (segment (start 170.326 93.3585) (end 168.999 94.6862) (width 0.25) (layer "F.Cu") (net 24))
 (segment (start 169.1205 94.8081) (end 168.999 94.6862) (width 0.25) (layer "F.Cu") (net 24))
 (segment (start 165.546 86.36) (end 168.41 89.224) (width 0.25) (layer "F.Cu") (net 24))
 (segment (start 168.292 93.98) (end 165.925 93.98) (width 0.25) (layer "F.Cu") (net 24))
 (segment (start 171.118 93.98) (end 171.118 95.8137) (width 0.25) (layer "F.Cu") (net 13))
 (segment (start 170.336 103.508) (end 170.037 103.808) (width 0.25) (layer "F.Cu") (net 13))
 (segment (start 170.356 104.791) (end 172.959 104.791) (width 0.25) (layer "F.Cu") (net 13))
 (segment (start 172.959 104.791) (end 173.61 104.14) (width 0.25) (layer "F.Cu") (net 13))
 (segment (start 170.336 99.6915) (end 170.336 103.508) (width 0.25) (layer "F.Cu") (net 13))
 (segment (start 171.1175 95.8132) (end 171.1175 93.98) (width 0.25) (layer "F.Cu") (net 13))
 (segment (start 171.118 95.8137) (end 171.1175 95.8132) (width 0.25) (layer "F.Cu") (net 13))
 (segment (start 170.037 99.3923) (end 170.336 99.6915) (width 0.25) (layer "F.Cu") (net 13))
 (segment (start 171.118 95.8137) (end 171.118 97.6475) (width 0.25) (layer "F.Cu") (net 13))
 (segment (start 170.037 98.7277) (end 170.037 99.3923) (width 0.25) (layer "F.Cu") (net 13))
 (segment (start 171.118 97.6475) (end 170.037 98.7277) (width 0.25) (layer "F.Cu") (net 13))
 (segment (start 170.037 104.472) (end 170.356 104.791) (width 0.25) (layer "F.Cu") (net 13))
 (segment (start 170.037 103.808) (end 170.037 104.472) (width 0.25) (layer "F.Cu") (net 13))
 (segment (start 160.845 91.0552) (end 160.845 91.44) (width 0.25) (layer "F.Cu") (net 14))
 (segment (start 165.107 88.0819) (end 163.818 88.0819) (width 0.25) (layer "F.Cu") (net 14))
 (segment (start 169.242 89.85) (end 166.875 89.85) (width 0.25) (layer "F.Cu") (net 14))
 (segment (start 166.875 89.85) (end 165.925 88.9) (width 0.25) (layer "F.Cu") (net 14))
 (segment (start 169.242 89.85) (end 169.2425 89.85) (width 0.25) (layer "F.Cu") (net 14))
 (segment (start 163.818 88.0819) (end 160.845 91.0552) (width 0.25) (layer "F.Cu") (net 14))
 (segment (start 165.925 88.9) (end 165.107 88.0819) (width 0.25) (layer "F.Cu") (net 14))
 (segment (start 171.118 88.9) (end 171.118 88.9237) (width 0.25) (layer "F.Cu") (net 15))
 (segment (start 173.61 93.98) (end 171.118 91.488) (width 0.25) (layer "F.Cu") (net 15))
 (segment (start 171.118 88.9237) (end 171.118 88.9475) (width 0.25) (layer "F.Cu") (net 15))
 (segment (start 171.118 88.9237) (end 171.1175 88.9232) (width 0.25) (layer "F.Cu") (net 15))
 (segment (start 171.118 91.488) (end 171.118 88.9475) (width 0.25) (layer "F.Cu") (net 15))
 (segment (start 171.1175 88.9232) (end 171.1175 88.9) (width 0.25) (layer "F.Cu") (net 15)))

